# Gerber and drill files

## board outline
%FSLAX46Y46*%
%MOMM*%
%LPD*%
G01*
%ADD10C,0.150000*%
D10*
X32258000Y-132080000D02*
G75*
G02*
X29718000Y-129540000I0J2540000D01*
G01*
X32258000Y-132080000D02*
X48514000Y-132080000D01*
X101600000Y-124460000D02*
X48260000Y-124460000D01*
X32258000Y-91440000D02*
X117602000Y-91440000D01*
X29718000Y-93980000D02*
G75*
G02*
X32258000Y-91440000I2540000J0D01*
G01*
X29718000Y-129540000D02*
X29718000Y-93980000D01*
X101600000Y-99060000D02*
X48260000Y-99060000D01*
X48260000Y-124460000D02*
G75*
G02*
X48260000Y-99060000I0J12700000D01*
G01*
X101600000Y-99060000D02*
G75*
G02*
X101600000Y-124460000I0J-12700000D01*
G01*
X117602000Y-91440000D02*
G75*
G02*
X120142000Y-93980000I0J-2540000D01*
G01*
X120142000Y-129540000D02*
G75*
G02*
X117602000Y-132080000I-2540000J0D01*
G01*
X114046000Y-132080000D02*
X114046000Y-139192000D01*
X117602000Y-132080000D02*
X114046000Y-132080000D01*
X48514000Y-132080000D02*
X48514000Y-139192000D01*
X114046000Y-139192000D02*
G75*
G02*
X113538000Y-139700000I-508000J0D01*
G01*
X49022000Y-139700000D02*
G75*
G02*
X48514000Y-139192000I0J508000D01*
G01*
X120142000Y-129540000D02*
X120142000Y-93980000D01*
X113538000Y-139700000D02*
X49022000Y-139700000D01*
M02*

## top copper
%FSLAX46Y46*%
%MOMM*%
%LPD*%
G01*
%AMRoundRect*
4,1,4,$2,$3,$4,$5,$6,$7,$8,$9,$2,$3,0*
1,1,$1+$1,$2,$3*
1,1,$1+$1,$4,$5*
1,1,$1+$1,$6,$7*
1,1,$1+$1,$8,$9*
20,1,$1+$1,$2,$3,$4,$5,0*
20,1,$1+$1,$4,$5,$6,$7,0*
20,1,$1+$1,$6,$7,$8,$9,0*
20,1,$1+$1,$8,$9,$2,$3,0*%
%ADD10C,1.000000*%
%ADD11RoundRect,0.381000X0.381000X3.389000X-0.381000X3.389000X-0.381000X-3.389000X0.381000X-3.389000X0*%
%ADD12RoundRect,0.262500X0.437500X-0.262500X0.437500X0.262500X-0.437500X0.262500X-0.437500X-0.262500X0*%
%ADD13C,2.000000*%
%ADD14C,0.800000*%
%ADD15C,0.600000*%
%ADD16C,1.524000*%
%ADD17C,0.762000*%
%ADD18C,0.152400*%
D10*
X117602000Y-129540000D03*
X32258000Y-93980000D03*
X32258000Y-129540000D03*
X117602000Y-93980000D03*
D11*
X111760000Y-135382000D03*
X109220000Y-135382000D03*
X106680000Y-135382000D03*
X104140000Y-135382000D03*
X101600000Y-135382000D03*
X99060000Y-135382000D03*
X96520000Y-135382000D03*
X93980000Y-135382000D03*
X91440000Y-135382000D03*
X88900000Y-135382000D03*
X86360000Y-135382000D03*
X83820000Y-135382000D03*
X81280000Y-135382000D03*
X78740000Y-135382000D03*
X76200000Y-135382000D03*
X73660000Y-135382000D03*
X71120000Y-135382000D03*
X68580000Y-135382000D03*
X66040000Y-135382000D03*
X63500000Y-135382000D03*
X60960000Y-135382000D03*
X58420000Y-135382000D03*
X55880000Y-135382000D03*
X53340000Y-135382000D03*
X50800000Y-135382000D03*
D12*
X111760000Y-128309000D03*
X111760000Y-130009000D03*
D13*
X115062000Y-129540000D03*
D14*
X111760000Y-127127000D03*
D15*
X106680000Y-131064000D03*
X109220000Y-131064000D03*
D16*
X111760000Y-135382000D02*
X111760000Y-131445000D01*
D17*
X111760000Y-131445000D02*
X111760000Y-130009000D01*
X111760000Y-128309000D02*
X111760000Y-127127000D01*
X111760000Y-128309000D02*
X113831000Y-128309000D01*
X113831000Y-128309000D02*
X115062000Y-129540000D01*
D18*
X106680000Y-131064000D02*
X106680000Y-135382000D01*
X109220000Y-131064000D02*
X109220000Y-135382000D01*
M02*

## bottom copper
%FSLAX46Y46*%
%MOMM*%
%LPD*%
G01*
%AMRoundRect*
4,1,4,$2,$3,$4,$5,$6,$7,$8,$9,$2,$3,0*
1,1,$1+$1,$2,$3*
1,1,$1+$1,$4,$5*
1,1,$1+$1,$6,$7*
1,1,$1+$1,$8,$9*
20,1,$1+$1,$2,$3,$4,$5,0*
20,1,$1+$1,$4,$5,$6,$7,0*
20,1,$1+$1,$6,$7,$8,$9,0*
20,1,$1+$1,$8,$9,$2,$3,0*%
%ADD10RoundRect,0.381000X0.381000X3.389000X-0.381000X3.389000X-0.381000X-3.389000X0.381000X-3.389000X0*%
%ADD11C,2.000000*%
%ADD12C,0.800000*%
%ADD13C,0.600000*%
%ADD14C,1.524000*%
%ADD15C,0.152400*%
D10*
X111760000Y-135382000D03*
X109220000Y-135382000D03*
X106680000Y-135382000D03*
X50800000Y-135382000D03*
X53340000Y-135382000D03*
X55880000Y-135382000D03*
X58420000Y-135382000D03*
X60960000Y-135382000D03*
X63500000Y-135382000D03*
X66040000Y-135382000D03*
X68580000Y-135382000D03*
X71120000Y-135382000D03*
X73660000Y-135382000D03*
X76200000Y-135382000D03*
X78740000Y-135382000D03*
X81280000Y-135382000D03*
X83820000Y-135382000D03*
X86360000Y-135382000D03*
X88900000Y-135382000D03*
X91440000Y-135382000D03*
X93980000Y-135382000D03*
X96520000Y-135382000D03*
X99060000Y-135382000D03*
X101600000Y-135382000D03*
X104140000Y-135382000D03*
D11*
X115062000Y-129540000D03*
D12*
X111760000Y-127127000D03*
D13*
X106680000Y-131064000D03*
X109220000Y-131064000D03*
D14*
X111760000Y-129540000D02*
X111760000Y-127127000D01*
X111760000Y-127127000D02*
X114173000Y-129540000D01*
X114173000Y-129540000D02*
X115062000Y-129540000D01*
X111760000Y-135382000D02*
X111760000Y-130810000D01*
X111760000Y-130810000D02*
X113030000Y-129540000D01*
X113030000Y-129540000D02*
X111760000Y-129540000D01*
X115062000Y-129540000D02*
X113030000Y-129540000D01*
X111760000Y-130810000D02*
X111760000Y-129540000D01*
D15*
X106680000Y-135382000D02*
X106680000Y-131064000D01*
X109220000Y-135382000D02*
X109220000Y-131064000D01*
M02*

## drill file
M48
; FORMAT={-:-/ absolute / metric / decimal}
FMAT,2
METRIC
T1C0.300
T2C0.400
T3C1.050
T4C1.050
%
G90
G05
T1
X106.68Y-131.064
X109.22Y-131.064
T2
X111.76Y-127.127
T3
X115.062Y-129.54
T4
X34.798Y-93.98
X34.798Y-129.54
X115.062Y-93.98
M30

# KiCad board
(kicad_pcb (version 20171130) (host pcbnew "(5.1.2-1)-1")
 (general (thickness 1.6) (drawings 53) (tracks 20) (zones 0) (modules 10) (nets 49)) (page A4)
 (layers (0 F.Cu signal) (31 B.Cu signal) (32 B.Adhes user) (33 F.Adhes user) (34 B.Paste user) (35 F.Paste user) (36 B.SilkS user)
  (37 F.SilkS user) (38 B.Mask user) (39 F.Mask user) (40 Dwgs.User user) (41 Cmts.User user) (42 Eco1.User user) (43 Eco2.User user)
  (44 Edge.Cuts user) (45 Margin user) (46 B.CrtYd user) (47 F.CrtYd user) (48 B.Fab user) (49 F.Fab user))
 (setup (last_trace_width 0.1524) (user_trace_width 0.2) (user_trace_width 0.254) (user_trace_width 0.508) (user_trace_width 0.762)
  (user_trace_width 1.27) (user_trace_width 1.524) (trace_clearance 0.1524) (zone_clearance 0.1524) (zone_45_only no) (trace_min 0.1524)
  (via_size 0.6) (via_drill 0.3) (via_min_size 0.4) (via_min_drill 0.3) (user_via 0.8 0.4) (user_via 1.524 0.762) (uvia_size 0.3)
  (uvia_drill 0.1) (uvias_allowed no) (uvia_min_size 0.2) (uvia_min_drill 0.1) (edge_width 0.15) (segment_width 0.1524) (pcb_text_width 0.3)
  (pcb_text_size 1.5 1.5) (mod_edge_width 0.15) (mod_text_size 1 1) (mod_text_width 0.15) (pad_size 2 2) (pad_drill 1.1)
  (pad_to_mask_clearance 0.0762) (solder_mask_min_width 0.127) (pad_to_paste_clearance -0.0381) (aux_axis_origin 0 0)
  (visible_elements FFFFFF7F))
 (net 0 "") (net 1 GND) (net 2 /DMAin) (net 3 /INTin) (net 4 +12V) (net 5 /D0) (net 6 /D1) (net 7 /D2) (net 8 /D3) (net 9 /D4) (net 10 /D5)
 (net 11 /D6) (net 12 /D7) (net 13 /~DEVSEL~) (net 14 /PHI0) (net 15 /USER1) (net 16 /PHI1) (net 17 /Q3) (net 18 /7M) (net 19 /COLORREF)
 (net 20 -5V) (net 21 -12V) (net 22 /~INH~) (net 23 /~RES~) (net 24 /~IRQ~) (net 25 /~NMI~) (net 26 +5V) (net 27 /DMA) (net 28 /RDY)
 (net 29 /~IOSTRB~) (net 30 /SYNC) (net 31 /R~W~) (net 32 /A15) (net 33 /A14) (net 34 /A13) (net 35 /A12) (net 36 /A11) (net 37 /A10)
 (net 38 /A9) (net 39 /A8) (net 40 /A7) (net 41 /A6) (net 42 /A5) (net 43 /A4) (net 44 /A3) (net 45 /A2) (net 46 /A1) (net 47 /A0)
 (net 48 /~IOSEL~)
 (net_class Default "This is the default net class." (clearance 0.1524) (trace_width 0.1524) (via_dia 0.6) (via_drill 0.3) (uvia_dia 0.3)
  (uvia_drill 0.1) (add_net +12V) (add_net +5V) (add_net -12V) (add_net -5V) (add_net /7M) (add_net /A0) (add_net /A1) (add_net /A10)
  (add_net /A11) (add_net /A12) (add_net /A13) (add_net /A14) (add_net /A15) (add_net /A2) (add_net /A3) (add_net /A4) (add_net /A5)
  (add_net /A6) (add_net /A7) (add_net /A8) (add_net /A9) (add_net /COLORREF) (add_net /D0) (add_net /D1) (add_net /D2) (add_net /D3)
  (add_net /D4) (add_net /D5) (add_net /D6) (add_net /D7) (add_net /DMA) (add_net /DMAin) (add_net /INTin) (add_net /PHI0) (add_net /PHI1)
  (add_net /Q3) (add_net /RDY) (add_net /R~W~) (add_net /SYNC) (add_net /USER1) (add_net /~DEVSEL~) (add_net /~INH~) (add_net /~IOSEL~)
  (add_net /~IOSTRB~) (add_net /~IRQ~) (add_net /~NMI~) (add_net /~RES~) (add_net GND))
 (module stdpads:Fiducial (layer F.Cu) (at 117.602 129.54)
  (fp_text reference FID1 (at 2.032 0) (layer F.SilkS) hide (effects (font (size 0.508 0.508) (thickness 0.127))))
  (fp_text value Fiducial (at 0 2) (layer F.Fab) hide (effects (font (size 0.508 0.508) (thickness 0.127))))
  (pad ~ smd circle (at 0 0) (size 1 1) (layers F.Cu F.Mask) (solder_mask_margin 0.5) (clearance 0.575)))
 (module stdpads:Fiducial (layer F.Cu) (at 32.258 93.98 180)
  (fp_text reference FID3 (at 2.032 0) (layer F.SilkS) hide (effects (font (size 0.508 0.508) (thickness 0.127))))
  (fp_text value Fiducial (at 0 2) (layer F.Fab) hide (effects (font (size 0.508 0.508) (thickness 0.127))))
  (pad ~ smd circle (at 0 0 180) (size 1 1) (layers F.Cu F.Mask) (solder_mask_margin 0.5) (clearance 0.575)))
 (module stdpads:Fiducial (layer F.Cu) (at 32.258 129.54 180)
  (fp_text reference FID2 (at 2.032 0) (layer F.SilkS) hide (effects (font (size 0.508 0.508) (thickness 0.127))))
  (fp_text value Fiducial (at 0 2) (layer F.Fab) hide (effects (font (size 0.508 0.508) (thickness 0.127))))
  (pad ~ smd circle (at 0 0 180) (size 1 1) (layers F.Cu F.Mask) (solder_mask_margin 0.5) (clearance 0.575)))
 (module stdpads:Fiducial (layer F.Cu) (at 117.602 93.98 270)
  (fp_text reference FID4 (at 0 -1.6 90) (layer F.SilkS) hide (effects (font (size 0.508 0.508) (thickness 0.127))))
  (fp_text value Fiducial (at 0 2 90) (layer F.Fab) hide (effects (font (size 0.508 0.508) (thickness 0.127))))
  (pad ~ smd circle (at 0 0 270) (size 1 1) (layers F.Cu F.Mask) (solder_mask_margin 0.5) (clearance 0.575)))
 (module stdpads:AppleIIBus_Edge (layer F.Cu) (at 81.28 135.382)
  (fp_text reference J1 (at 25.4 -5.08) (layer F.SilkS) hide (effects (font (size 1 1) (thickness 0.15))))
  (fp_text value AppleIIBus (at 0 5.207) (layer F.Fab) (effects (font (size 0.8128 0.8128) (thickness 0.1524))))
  (pad 26 smd roundrect (at 30.48 0 180) (size 1.524 7.54) (layers B.Cu B.Mask) (roundrect_rratio 0.25) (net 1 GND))
  (pad 27 smd roundrect (at 27.94 0 180) (size 1.524 7.54) (layers B.Cu B.Mask) (roundrect_rratio 0.25) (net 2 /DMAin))
  (pad 28 smd roundrect (at 25.4 0 180) (size 1.524 7.54) (layers B.Cu B.Mask) (roundrect_rratio 0.25) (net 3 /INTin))
  (pad 50 smd roundrect (at -30.48 0 180) (size 1.524 7.54) (layers B.Cu B.Mask) (roundrect_rratio 0.25) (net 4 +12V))
  (pad 49 smd roundrect (at -27.94 0 180) (size 1.524 7.54) (layers B.Cu B.Mask) (roundrect_rratio 0.25) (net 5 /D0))
  (pad 48 smd roundrect (at -25.4 0 180) (size 1.524 7.54) (layers B.Cu B.Mask) (roundrect_rratio 0.25) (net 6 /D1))
  (pad 47 smd roundrect (at -22.86 0 180) (size 1.524 7.54) (layers B.Cu B.Mask) (roundrect_rratio 0.25) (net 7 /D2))
  (pad 46 smd roundrect (at -20.32 0 180) (size 1.524 7.54) (layers B.Cu B.Mask) (roundrect_rratio 0.25) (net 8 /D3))
  (pad 45 smd roundrect (at -17.78 0 180) (size 1.524 7.54) (layers B.Cu B.Mask) (roundrect_rratio 0.25) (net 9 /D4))
  (pad 44 smd roundrect (at -15.24 0 180) (size 1.524 7.54) (layers B.Cu B.Mask) (roundrect_rratio 0.25) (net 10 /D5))
  (pad 43 smd roundrect (at -12.7 0 180) (size 1.524 7.54) (layers B.Cu B.Mask) (roundrect_rratio 0.25) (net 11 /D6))
  (pad 42 smd roundrect (at -10.16 0 180) (size 1.524 7.54) (layers B.Cu B.Mask) (roundrect_rratio 0.25) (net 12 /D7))
  (pad 41 smd roundrect (at -7.62 0 180) (size 1.524 7.54) (layers B.Cu B.Mask) (roundrect_rratio 0.25) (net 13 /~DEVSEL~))
  (pad 40 smd roundrect (at -5.08 0 180) (size 1.524 7.54) (layers B.Cu B.Mask) (roundrect_rratio 0.25) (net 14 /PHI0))
  (pad 39 smd roundrect (at -2.54 0 180) (size 1.524 7.54) (layers B.Cu B.Mask) (roundrect_rratio 0.25) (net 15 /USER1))
  (pad 38 smd roundrect (at 0 0 180) (size 1.524 7.54) (layers B.Cu B.Mask) (roundrect_rratio 0.25) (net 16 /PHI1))
  (pad 37 smd roundrect (at 2.54 0 180) (size 1.524 7.54) (layers B.Cu B.Mask) (roundrect_rratio 0.25) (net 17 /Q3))
  (pad 36 smd roundrect (at 5.08 0 180) (size 1.524 7.54) (layers B.Cu B.Mask) (roundrect_rratio 0.25) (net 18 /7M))
  (pad 35 smd roundrect (at 7.62 0 180) (size 1.524 7.54) (layers B.Cu B.Mask) (roundrect_rratio 0.25) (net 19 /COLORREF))
  (pad 34 smd roundrect (at 10.16 0 180) (size 1.524 7.54) (layers B.Cu B.Mask) (roundrect_rratio 0.25) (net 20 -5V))
  (pad 33 smd roundrect (at 12.7 0 180) (size 1.524 7.54) (layers B.Cu B.Mask) (roundrect_rratio 0.25) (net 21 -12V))
  (pad 32 smd roundrect (at 15.24 0 180) (size 1.524 7.54) (layers B.Cu B.Mask) (roundrect_rratio 0.25) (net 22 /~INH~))
  (pad 31 smd roundrect (at 17.78 0 180) (size 1.524 7.54) (layers B.Cu B.Mask) (roundrect_rratio 0.25) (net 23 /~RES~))
  (pad 30 smd roundrect (at 20.32 0 180) (size 1.524 7.54) (layers B.Cu B.Mask) (roundrect_rratio 0.25) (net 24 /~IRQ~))
  (pad 29 smd roundrect (at 22.86 0 180) (size 1.524 7.54) (layers B.Cu B.Mask) (roundrect_rratio 0.25) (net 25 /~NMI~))
  (pad 25 smd roundrect (at 30.48 0 180) (size 1.524 7.54) (layers F.Cu F.Mask) (roundrect_rratio 0.25) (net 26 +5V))
  (pad 24 smd roundrect (at 27.94 0 180) (size 1.524 7.54) (layers F.Cu F.Mask) (roundrect_rratio 0.25) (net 2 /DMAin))
  (pad 23 smd roundrect (at 25.4 0 180) (size 1.524 7.54) (layers F.Cu F.Mask) (roundrect_rratio 0.25) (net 3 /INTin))
  (pad 22 smd roundrect (at 22.86 0 180) (size 1.524 7.54) (layers F.Cu F.Mask) (roundrect_rratio 0.25) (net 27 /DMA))
  (pad 21 smd roundrect (at 20.32 0 180) (size 1.524 7.54) (layers F.Cu F.Mask) (roundrect_rratio 0.25) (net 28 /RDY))
  (pad 20 smd roundrect (at 17.78 0 180) (size 1.524 7.54) (layers F.Cu F.Mask) (roundrect_rratio 0.25) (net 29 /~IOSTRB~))
  (pad 19 smd roundrect (at 15.24 0 180) (size 1.524 7.54) (layers F.Cu F.Mask) (roundrect_rratio 0.25) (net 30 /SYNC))
  (pad 18 smd roundrect (at 12.7 0 180) (size 1.524 7.54) (layers F.Cu F.Mask) (roundrect_rratio 0.25) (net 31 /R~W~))
  (pad 17 smd roundrect (at 10.16 0 180) (size 1.524 7.54) (layers F.Cu F.Mask) (roundrect_rratio 0.25) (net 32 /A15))
  (pad 16 smd roundrect (at 7.62 0 180) (size 1.524 7.54) (layers F.Cu F.Mask) (roundrect_rratio 0.25) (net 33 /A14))
  (pad 15 smd roundrect (at 5.08 0 180) (size 1.524 7.54) (layers F.Cu F.Mask) (roundrect_rratio 0.25) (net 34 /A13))
  (pad 14 smd roundrect (at 2.54 0 180) (size 1.524 7.54) (layers F.Cu F.Mask) (roundrect_rratio 0.25) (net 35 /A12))
  (pad 13 smd roundrect (at 0 0 180) (size 1.524 7.54) (layers F.Cu F.Mask) (roundrect_rratio 0.25) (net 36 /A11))
  (pad 12 smd roundrect (at -2.54 0 180) (size 1.524 7.54) (layers F.Cu F.Mask) (roundrect_rratio 0.25) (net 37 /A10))
  (pad 11 smd roundrect (at -5.08 0 180) (size 1.524 7.54) (layers F.Cu F.Mask) (roundrect_rratio 0.25) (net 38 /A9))
  (pad 10 smd roundrect (at -7.62 0 180) (size 1.524 7.54) (layers F.Cu F.Mask) (roundrect_rratio 0.25) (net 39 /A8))
  (pad 9 smd roundrect (at -10.16 0 180) (size 1.524 7.54) (layers F.Cu F.Mask) (roundrect_rratio 0.25) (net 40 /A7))
  (pad 8 smd roundrect (at -12.7 0 180) (size 1.524 7.54) (layers F.Cu F.Mask) (roundrect_rratio 0.25) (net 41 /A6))
  (pad 7 smd roundrect (at -15.24 0 180) (size 1.524 7.54) (layers F.Cu F.Mask) (roundrect_rratio 0.25) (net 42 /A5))
  (pad 6 smd roundrect (at -17.78 0 180) (size 1.524 7.54) (layers F.Cu F.Mask) (roundrect_rratio 0.25) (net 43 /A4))
  (pad 5 smd roundrect (at -20.32 0 180) (size 1.524 7.54) (layers F.Cu F.Mask) (roundrect_rratio 0.25) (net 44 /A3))
  (pad 4 smd roundrect (at -22.86 0 180) (size 1.524 7.54) (layers F.Cu F.Mask) (roundrect_rratio 0.25) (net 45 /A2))
  (pad 3 smd roundrect (at -25.4 0 180) (size 1.524 7.54) (layers F.Cu F.Mask) (roundrect_rratio 0.25) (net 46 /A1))
  (pad 2 smd roundrect (at -27.94 0 180) (size 1.524 7.54) (layers F.Cu F.Mask) (roundrect_rratio 0.25) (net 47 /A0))
  (pad 1 smd roundrect (at -30.48 0 180) (size 1.524 7.54) (layers F.Cu F.Mask) (roundrect_rratio 0.25) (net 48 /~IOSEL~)))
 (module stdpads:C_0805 (layer F.Cu) (at 111.76 129.159 90)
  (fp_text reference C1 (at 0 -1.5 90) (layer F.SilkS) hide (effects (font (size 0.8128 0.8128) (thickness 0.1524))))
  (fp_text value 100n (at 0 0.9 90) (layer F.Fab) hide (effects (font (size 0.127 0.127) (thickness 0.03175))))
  (pad 2 smd roundrect (at 0.85 0 90) (size 1.05 1.4) (layers F.Cu F.Paste F.Mask) (roundrect_rratio 0.25) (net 1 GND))
  (pad 1 smd roundrect (at -0.85 0 90) (size 1.05 1.4) (layers F.Cu F.Paste F.Mask) (roundrect_rratio 0.25) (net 26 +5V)))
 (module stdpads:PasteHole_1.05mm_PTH (layer F.Cu) (at 115.062 129.54) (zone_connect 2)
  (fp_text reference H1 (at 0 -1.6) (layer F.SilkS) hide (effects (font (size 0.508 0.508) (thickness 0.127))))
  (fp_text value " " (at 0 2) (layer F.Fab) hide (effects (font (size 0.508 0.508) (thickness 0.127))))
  (pad 1 thru_hole circle (at 0 0) (size 2 2) (drill 1.05) (layers *.Cu *.Mask) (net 1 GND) (zone_connect 2)))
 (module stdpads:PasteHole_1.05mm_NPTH (layer F.Cu) (at 34.798 129.54 180)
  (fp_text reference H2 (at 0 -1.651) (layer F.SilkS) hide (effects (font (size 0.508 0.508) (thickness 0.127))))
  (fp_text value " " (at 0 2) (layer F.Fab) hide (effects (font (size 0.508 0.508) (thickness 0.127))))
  (pad "" np_thru_hole oval (at 0 0 180) (size 1.05 1.05) (drill 1.05) (layers *.Cu *.Mask)))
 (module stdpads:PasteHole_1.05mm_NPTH (layer F.Cu) (at 34.798 93.98 180)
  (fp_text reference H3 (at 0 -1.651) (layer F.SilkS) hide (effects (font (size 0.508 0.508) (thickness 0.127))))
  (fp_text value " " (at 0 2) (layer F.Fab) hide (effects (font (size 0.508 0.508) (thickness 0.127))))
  (pad "" np_thru_hole oval (at 0 0 180) (size 1.05 1.05) (drill 1.05) (layers *.Cu *.Mask)))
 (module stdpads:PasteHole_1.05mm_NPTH (layer F.Cu) (at 115.062 93.98 270)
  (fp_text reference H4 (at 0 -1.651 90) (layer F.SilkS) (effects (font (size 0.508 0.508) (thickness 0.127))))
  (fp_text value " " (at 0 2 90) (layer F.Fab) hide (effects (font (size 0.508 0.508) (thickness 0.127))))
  (pad "" np_thru_hole oval (at 0 0 270) (size 1.05 1.05) (drill 1.05) (layers *.Cu *.Mask)))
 (gr_arc (start 32.258 129.54) (end 29.718 129.54) (angle -90) (layer Edge.Cuts) (width 0.15))
 (gr_line (start 32.258 132.08) (end 48.514 132.08) (layer Edge.Cuts) (width 0.15))
 (gr_line (start 101.6 124.46) (end 48.26 124.46) (layer Edge.Cuts) (width 0.15))
 (gr_line (start 32.258 91.44) (end 117.602 91.44) (layer Edge.Cuts) (width 0.15))
 (gr_arc (start 32.258 93.98) (end 32.258 91.44) (angle -90) (layer Edge.Cuts) (width 0.15))
 (gr_line (start 29.718 129.54) (end 29.718 93.98) (layer Edge.Cuts) (width 0.15))
 (gr_line (start 101.6 99.06) (end 48.26 99.06) (layer Edge.Cuts) (width 0.15))
 (gr_arc (start 48.26 111.76) (end 48.26 99.06) (angle -180) (layer Edge.Cuts) (width 0.15))
 (gr_arc (start 101.6 111.76) (end 101.6 124.46) (angle -180) (layer Edge.Cuts) (width 0.15))
 (gr_arc (start 117.602 93.98) (end 120.142 93.98) (angle -90) (layer Edge.Cuts) (width 0.15))
 (gr_arc (start 117.602 129.54) (end 117.602 132.08) (angle -90) (layer Edge.Cuts) (width 0.15))
 (gr_line (start 114.046 132.08) (end 114.046 139.192) (layer Edge.Cuts) (width 0.15))
 (gr_line (start 117.602 132.08) (end 114.046 132.08) (layer Edge.Cuts) (width 0.15))
 (gr_line (start 48.514 132.08) (end 48.514 139.192) (layer Edge.Cuts) (width 0.15))
 (gr_arc (start 113.538 139.192) (end 113.538 139.7) (angle -90) (layer Edge.Cuts) (width 0.15))
 (gr_arc (start 49.022 139.192) (end 48.514 139.192) (angle -90) (layer Edge.Cuts) (width 0.15))
 (gr_line (start 120.142 129.54) (end 120.142 93.98) (angle 90) (layer Edge.Cuts) (width 0.15))
 (gr_line (start 113.538 139.7) (end 49.022 139.7) (layer Edge.Cuts) (width 0.15))
 (segment (start 111.76 135.382) (end 111.76 131.445) (width 1.524) (layer F.Cu) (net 26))
 (segment (start 111.76 131.445) (end 111.76 130.009) (width 0.762) (layer F.Cu) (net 26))
 (via (at 111.76 127.127) (size 0.8) (drill 0.4) (layers F.Cu B.Cu) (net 1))
 (segment (start 111.76 128.309) (end 111.76 127.127) (width 0.762) (layer F.Cu) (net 1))
 (segment (start 111.76 129.54) (end 111.76 127.127) (width 1.524) (layer B.Cu) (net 1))
 (segment (start 111.76 128.309) (end 113.831 128.309) (width 0.762) (layer F.Cu) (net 1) (status 400000))
 (segment (start 113.831 128.309) (end 115.062 129.54) (width 0.762) (layer F.Cu) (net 1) (status 800000))
 (segment (start 111.76 127.127) (end 114.173 129.54) (width 1.524) (layer B.Cu) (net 1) (status 800000))
 (segment (start 114.173 129.54) (end 115.062 129.54) (width 1.524) (layer B.Cu) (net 1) (status C00000))
 (segment (start 111.76 135.382) (end 111.76 130.81) (width 1.524) (layer B.Cu) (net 1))
 (segment (start 111.76 130.81) (end 113.03 129.54) (width 1.524) (layer B.Cu) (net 1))
 (segment (start 113.03 129.54) (end 111.76 129.54) (width 1.524) (layer B.Cu) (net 1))
 (segment (start 115.062 129.54) (end 113.03 129.54) (width 1.524) (layer B.Cu) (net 1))
 (segment (start 111.76 130.81) (end 111.76 129.54) (width 1.524) (layer B.Cu) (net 1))
 (segment (start 106.68 135.382) (end 106.68 131.064) (width 0.1524) (layer B.Cu) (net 3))
 (via (at 106.68 131.064) (size 0.6) (drill 0.3) (layers F.Cu B.Cu) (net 3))
 (segment (start 106.68 131.064) (end 106.68 135.382) (width 0.1524) (layer F.Cu) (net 3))
 (via (at 109.22 131.064) (size 0.6) (drill 0.3) (layers F.Cu B.Cu) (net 2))
 (segment (start 109.22 135.382) (end 109.22 131.064) (width 0.1524) (layer B.Cu) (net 2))
 (segment (start 109.22 131.064) (end 109.22 135.382) (width 0.1524) (layer F.Cu) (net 2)))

